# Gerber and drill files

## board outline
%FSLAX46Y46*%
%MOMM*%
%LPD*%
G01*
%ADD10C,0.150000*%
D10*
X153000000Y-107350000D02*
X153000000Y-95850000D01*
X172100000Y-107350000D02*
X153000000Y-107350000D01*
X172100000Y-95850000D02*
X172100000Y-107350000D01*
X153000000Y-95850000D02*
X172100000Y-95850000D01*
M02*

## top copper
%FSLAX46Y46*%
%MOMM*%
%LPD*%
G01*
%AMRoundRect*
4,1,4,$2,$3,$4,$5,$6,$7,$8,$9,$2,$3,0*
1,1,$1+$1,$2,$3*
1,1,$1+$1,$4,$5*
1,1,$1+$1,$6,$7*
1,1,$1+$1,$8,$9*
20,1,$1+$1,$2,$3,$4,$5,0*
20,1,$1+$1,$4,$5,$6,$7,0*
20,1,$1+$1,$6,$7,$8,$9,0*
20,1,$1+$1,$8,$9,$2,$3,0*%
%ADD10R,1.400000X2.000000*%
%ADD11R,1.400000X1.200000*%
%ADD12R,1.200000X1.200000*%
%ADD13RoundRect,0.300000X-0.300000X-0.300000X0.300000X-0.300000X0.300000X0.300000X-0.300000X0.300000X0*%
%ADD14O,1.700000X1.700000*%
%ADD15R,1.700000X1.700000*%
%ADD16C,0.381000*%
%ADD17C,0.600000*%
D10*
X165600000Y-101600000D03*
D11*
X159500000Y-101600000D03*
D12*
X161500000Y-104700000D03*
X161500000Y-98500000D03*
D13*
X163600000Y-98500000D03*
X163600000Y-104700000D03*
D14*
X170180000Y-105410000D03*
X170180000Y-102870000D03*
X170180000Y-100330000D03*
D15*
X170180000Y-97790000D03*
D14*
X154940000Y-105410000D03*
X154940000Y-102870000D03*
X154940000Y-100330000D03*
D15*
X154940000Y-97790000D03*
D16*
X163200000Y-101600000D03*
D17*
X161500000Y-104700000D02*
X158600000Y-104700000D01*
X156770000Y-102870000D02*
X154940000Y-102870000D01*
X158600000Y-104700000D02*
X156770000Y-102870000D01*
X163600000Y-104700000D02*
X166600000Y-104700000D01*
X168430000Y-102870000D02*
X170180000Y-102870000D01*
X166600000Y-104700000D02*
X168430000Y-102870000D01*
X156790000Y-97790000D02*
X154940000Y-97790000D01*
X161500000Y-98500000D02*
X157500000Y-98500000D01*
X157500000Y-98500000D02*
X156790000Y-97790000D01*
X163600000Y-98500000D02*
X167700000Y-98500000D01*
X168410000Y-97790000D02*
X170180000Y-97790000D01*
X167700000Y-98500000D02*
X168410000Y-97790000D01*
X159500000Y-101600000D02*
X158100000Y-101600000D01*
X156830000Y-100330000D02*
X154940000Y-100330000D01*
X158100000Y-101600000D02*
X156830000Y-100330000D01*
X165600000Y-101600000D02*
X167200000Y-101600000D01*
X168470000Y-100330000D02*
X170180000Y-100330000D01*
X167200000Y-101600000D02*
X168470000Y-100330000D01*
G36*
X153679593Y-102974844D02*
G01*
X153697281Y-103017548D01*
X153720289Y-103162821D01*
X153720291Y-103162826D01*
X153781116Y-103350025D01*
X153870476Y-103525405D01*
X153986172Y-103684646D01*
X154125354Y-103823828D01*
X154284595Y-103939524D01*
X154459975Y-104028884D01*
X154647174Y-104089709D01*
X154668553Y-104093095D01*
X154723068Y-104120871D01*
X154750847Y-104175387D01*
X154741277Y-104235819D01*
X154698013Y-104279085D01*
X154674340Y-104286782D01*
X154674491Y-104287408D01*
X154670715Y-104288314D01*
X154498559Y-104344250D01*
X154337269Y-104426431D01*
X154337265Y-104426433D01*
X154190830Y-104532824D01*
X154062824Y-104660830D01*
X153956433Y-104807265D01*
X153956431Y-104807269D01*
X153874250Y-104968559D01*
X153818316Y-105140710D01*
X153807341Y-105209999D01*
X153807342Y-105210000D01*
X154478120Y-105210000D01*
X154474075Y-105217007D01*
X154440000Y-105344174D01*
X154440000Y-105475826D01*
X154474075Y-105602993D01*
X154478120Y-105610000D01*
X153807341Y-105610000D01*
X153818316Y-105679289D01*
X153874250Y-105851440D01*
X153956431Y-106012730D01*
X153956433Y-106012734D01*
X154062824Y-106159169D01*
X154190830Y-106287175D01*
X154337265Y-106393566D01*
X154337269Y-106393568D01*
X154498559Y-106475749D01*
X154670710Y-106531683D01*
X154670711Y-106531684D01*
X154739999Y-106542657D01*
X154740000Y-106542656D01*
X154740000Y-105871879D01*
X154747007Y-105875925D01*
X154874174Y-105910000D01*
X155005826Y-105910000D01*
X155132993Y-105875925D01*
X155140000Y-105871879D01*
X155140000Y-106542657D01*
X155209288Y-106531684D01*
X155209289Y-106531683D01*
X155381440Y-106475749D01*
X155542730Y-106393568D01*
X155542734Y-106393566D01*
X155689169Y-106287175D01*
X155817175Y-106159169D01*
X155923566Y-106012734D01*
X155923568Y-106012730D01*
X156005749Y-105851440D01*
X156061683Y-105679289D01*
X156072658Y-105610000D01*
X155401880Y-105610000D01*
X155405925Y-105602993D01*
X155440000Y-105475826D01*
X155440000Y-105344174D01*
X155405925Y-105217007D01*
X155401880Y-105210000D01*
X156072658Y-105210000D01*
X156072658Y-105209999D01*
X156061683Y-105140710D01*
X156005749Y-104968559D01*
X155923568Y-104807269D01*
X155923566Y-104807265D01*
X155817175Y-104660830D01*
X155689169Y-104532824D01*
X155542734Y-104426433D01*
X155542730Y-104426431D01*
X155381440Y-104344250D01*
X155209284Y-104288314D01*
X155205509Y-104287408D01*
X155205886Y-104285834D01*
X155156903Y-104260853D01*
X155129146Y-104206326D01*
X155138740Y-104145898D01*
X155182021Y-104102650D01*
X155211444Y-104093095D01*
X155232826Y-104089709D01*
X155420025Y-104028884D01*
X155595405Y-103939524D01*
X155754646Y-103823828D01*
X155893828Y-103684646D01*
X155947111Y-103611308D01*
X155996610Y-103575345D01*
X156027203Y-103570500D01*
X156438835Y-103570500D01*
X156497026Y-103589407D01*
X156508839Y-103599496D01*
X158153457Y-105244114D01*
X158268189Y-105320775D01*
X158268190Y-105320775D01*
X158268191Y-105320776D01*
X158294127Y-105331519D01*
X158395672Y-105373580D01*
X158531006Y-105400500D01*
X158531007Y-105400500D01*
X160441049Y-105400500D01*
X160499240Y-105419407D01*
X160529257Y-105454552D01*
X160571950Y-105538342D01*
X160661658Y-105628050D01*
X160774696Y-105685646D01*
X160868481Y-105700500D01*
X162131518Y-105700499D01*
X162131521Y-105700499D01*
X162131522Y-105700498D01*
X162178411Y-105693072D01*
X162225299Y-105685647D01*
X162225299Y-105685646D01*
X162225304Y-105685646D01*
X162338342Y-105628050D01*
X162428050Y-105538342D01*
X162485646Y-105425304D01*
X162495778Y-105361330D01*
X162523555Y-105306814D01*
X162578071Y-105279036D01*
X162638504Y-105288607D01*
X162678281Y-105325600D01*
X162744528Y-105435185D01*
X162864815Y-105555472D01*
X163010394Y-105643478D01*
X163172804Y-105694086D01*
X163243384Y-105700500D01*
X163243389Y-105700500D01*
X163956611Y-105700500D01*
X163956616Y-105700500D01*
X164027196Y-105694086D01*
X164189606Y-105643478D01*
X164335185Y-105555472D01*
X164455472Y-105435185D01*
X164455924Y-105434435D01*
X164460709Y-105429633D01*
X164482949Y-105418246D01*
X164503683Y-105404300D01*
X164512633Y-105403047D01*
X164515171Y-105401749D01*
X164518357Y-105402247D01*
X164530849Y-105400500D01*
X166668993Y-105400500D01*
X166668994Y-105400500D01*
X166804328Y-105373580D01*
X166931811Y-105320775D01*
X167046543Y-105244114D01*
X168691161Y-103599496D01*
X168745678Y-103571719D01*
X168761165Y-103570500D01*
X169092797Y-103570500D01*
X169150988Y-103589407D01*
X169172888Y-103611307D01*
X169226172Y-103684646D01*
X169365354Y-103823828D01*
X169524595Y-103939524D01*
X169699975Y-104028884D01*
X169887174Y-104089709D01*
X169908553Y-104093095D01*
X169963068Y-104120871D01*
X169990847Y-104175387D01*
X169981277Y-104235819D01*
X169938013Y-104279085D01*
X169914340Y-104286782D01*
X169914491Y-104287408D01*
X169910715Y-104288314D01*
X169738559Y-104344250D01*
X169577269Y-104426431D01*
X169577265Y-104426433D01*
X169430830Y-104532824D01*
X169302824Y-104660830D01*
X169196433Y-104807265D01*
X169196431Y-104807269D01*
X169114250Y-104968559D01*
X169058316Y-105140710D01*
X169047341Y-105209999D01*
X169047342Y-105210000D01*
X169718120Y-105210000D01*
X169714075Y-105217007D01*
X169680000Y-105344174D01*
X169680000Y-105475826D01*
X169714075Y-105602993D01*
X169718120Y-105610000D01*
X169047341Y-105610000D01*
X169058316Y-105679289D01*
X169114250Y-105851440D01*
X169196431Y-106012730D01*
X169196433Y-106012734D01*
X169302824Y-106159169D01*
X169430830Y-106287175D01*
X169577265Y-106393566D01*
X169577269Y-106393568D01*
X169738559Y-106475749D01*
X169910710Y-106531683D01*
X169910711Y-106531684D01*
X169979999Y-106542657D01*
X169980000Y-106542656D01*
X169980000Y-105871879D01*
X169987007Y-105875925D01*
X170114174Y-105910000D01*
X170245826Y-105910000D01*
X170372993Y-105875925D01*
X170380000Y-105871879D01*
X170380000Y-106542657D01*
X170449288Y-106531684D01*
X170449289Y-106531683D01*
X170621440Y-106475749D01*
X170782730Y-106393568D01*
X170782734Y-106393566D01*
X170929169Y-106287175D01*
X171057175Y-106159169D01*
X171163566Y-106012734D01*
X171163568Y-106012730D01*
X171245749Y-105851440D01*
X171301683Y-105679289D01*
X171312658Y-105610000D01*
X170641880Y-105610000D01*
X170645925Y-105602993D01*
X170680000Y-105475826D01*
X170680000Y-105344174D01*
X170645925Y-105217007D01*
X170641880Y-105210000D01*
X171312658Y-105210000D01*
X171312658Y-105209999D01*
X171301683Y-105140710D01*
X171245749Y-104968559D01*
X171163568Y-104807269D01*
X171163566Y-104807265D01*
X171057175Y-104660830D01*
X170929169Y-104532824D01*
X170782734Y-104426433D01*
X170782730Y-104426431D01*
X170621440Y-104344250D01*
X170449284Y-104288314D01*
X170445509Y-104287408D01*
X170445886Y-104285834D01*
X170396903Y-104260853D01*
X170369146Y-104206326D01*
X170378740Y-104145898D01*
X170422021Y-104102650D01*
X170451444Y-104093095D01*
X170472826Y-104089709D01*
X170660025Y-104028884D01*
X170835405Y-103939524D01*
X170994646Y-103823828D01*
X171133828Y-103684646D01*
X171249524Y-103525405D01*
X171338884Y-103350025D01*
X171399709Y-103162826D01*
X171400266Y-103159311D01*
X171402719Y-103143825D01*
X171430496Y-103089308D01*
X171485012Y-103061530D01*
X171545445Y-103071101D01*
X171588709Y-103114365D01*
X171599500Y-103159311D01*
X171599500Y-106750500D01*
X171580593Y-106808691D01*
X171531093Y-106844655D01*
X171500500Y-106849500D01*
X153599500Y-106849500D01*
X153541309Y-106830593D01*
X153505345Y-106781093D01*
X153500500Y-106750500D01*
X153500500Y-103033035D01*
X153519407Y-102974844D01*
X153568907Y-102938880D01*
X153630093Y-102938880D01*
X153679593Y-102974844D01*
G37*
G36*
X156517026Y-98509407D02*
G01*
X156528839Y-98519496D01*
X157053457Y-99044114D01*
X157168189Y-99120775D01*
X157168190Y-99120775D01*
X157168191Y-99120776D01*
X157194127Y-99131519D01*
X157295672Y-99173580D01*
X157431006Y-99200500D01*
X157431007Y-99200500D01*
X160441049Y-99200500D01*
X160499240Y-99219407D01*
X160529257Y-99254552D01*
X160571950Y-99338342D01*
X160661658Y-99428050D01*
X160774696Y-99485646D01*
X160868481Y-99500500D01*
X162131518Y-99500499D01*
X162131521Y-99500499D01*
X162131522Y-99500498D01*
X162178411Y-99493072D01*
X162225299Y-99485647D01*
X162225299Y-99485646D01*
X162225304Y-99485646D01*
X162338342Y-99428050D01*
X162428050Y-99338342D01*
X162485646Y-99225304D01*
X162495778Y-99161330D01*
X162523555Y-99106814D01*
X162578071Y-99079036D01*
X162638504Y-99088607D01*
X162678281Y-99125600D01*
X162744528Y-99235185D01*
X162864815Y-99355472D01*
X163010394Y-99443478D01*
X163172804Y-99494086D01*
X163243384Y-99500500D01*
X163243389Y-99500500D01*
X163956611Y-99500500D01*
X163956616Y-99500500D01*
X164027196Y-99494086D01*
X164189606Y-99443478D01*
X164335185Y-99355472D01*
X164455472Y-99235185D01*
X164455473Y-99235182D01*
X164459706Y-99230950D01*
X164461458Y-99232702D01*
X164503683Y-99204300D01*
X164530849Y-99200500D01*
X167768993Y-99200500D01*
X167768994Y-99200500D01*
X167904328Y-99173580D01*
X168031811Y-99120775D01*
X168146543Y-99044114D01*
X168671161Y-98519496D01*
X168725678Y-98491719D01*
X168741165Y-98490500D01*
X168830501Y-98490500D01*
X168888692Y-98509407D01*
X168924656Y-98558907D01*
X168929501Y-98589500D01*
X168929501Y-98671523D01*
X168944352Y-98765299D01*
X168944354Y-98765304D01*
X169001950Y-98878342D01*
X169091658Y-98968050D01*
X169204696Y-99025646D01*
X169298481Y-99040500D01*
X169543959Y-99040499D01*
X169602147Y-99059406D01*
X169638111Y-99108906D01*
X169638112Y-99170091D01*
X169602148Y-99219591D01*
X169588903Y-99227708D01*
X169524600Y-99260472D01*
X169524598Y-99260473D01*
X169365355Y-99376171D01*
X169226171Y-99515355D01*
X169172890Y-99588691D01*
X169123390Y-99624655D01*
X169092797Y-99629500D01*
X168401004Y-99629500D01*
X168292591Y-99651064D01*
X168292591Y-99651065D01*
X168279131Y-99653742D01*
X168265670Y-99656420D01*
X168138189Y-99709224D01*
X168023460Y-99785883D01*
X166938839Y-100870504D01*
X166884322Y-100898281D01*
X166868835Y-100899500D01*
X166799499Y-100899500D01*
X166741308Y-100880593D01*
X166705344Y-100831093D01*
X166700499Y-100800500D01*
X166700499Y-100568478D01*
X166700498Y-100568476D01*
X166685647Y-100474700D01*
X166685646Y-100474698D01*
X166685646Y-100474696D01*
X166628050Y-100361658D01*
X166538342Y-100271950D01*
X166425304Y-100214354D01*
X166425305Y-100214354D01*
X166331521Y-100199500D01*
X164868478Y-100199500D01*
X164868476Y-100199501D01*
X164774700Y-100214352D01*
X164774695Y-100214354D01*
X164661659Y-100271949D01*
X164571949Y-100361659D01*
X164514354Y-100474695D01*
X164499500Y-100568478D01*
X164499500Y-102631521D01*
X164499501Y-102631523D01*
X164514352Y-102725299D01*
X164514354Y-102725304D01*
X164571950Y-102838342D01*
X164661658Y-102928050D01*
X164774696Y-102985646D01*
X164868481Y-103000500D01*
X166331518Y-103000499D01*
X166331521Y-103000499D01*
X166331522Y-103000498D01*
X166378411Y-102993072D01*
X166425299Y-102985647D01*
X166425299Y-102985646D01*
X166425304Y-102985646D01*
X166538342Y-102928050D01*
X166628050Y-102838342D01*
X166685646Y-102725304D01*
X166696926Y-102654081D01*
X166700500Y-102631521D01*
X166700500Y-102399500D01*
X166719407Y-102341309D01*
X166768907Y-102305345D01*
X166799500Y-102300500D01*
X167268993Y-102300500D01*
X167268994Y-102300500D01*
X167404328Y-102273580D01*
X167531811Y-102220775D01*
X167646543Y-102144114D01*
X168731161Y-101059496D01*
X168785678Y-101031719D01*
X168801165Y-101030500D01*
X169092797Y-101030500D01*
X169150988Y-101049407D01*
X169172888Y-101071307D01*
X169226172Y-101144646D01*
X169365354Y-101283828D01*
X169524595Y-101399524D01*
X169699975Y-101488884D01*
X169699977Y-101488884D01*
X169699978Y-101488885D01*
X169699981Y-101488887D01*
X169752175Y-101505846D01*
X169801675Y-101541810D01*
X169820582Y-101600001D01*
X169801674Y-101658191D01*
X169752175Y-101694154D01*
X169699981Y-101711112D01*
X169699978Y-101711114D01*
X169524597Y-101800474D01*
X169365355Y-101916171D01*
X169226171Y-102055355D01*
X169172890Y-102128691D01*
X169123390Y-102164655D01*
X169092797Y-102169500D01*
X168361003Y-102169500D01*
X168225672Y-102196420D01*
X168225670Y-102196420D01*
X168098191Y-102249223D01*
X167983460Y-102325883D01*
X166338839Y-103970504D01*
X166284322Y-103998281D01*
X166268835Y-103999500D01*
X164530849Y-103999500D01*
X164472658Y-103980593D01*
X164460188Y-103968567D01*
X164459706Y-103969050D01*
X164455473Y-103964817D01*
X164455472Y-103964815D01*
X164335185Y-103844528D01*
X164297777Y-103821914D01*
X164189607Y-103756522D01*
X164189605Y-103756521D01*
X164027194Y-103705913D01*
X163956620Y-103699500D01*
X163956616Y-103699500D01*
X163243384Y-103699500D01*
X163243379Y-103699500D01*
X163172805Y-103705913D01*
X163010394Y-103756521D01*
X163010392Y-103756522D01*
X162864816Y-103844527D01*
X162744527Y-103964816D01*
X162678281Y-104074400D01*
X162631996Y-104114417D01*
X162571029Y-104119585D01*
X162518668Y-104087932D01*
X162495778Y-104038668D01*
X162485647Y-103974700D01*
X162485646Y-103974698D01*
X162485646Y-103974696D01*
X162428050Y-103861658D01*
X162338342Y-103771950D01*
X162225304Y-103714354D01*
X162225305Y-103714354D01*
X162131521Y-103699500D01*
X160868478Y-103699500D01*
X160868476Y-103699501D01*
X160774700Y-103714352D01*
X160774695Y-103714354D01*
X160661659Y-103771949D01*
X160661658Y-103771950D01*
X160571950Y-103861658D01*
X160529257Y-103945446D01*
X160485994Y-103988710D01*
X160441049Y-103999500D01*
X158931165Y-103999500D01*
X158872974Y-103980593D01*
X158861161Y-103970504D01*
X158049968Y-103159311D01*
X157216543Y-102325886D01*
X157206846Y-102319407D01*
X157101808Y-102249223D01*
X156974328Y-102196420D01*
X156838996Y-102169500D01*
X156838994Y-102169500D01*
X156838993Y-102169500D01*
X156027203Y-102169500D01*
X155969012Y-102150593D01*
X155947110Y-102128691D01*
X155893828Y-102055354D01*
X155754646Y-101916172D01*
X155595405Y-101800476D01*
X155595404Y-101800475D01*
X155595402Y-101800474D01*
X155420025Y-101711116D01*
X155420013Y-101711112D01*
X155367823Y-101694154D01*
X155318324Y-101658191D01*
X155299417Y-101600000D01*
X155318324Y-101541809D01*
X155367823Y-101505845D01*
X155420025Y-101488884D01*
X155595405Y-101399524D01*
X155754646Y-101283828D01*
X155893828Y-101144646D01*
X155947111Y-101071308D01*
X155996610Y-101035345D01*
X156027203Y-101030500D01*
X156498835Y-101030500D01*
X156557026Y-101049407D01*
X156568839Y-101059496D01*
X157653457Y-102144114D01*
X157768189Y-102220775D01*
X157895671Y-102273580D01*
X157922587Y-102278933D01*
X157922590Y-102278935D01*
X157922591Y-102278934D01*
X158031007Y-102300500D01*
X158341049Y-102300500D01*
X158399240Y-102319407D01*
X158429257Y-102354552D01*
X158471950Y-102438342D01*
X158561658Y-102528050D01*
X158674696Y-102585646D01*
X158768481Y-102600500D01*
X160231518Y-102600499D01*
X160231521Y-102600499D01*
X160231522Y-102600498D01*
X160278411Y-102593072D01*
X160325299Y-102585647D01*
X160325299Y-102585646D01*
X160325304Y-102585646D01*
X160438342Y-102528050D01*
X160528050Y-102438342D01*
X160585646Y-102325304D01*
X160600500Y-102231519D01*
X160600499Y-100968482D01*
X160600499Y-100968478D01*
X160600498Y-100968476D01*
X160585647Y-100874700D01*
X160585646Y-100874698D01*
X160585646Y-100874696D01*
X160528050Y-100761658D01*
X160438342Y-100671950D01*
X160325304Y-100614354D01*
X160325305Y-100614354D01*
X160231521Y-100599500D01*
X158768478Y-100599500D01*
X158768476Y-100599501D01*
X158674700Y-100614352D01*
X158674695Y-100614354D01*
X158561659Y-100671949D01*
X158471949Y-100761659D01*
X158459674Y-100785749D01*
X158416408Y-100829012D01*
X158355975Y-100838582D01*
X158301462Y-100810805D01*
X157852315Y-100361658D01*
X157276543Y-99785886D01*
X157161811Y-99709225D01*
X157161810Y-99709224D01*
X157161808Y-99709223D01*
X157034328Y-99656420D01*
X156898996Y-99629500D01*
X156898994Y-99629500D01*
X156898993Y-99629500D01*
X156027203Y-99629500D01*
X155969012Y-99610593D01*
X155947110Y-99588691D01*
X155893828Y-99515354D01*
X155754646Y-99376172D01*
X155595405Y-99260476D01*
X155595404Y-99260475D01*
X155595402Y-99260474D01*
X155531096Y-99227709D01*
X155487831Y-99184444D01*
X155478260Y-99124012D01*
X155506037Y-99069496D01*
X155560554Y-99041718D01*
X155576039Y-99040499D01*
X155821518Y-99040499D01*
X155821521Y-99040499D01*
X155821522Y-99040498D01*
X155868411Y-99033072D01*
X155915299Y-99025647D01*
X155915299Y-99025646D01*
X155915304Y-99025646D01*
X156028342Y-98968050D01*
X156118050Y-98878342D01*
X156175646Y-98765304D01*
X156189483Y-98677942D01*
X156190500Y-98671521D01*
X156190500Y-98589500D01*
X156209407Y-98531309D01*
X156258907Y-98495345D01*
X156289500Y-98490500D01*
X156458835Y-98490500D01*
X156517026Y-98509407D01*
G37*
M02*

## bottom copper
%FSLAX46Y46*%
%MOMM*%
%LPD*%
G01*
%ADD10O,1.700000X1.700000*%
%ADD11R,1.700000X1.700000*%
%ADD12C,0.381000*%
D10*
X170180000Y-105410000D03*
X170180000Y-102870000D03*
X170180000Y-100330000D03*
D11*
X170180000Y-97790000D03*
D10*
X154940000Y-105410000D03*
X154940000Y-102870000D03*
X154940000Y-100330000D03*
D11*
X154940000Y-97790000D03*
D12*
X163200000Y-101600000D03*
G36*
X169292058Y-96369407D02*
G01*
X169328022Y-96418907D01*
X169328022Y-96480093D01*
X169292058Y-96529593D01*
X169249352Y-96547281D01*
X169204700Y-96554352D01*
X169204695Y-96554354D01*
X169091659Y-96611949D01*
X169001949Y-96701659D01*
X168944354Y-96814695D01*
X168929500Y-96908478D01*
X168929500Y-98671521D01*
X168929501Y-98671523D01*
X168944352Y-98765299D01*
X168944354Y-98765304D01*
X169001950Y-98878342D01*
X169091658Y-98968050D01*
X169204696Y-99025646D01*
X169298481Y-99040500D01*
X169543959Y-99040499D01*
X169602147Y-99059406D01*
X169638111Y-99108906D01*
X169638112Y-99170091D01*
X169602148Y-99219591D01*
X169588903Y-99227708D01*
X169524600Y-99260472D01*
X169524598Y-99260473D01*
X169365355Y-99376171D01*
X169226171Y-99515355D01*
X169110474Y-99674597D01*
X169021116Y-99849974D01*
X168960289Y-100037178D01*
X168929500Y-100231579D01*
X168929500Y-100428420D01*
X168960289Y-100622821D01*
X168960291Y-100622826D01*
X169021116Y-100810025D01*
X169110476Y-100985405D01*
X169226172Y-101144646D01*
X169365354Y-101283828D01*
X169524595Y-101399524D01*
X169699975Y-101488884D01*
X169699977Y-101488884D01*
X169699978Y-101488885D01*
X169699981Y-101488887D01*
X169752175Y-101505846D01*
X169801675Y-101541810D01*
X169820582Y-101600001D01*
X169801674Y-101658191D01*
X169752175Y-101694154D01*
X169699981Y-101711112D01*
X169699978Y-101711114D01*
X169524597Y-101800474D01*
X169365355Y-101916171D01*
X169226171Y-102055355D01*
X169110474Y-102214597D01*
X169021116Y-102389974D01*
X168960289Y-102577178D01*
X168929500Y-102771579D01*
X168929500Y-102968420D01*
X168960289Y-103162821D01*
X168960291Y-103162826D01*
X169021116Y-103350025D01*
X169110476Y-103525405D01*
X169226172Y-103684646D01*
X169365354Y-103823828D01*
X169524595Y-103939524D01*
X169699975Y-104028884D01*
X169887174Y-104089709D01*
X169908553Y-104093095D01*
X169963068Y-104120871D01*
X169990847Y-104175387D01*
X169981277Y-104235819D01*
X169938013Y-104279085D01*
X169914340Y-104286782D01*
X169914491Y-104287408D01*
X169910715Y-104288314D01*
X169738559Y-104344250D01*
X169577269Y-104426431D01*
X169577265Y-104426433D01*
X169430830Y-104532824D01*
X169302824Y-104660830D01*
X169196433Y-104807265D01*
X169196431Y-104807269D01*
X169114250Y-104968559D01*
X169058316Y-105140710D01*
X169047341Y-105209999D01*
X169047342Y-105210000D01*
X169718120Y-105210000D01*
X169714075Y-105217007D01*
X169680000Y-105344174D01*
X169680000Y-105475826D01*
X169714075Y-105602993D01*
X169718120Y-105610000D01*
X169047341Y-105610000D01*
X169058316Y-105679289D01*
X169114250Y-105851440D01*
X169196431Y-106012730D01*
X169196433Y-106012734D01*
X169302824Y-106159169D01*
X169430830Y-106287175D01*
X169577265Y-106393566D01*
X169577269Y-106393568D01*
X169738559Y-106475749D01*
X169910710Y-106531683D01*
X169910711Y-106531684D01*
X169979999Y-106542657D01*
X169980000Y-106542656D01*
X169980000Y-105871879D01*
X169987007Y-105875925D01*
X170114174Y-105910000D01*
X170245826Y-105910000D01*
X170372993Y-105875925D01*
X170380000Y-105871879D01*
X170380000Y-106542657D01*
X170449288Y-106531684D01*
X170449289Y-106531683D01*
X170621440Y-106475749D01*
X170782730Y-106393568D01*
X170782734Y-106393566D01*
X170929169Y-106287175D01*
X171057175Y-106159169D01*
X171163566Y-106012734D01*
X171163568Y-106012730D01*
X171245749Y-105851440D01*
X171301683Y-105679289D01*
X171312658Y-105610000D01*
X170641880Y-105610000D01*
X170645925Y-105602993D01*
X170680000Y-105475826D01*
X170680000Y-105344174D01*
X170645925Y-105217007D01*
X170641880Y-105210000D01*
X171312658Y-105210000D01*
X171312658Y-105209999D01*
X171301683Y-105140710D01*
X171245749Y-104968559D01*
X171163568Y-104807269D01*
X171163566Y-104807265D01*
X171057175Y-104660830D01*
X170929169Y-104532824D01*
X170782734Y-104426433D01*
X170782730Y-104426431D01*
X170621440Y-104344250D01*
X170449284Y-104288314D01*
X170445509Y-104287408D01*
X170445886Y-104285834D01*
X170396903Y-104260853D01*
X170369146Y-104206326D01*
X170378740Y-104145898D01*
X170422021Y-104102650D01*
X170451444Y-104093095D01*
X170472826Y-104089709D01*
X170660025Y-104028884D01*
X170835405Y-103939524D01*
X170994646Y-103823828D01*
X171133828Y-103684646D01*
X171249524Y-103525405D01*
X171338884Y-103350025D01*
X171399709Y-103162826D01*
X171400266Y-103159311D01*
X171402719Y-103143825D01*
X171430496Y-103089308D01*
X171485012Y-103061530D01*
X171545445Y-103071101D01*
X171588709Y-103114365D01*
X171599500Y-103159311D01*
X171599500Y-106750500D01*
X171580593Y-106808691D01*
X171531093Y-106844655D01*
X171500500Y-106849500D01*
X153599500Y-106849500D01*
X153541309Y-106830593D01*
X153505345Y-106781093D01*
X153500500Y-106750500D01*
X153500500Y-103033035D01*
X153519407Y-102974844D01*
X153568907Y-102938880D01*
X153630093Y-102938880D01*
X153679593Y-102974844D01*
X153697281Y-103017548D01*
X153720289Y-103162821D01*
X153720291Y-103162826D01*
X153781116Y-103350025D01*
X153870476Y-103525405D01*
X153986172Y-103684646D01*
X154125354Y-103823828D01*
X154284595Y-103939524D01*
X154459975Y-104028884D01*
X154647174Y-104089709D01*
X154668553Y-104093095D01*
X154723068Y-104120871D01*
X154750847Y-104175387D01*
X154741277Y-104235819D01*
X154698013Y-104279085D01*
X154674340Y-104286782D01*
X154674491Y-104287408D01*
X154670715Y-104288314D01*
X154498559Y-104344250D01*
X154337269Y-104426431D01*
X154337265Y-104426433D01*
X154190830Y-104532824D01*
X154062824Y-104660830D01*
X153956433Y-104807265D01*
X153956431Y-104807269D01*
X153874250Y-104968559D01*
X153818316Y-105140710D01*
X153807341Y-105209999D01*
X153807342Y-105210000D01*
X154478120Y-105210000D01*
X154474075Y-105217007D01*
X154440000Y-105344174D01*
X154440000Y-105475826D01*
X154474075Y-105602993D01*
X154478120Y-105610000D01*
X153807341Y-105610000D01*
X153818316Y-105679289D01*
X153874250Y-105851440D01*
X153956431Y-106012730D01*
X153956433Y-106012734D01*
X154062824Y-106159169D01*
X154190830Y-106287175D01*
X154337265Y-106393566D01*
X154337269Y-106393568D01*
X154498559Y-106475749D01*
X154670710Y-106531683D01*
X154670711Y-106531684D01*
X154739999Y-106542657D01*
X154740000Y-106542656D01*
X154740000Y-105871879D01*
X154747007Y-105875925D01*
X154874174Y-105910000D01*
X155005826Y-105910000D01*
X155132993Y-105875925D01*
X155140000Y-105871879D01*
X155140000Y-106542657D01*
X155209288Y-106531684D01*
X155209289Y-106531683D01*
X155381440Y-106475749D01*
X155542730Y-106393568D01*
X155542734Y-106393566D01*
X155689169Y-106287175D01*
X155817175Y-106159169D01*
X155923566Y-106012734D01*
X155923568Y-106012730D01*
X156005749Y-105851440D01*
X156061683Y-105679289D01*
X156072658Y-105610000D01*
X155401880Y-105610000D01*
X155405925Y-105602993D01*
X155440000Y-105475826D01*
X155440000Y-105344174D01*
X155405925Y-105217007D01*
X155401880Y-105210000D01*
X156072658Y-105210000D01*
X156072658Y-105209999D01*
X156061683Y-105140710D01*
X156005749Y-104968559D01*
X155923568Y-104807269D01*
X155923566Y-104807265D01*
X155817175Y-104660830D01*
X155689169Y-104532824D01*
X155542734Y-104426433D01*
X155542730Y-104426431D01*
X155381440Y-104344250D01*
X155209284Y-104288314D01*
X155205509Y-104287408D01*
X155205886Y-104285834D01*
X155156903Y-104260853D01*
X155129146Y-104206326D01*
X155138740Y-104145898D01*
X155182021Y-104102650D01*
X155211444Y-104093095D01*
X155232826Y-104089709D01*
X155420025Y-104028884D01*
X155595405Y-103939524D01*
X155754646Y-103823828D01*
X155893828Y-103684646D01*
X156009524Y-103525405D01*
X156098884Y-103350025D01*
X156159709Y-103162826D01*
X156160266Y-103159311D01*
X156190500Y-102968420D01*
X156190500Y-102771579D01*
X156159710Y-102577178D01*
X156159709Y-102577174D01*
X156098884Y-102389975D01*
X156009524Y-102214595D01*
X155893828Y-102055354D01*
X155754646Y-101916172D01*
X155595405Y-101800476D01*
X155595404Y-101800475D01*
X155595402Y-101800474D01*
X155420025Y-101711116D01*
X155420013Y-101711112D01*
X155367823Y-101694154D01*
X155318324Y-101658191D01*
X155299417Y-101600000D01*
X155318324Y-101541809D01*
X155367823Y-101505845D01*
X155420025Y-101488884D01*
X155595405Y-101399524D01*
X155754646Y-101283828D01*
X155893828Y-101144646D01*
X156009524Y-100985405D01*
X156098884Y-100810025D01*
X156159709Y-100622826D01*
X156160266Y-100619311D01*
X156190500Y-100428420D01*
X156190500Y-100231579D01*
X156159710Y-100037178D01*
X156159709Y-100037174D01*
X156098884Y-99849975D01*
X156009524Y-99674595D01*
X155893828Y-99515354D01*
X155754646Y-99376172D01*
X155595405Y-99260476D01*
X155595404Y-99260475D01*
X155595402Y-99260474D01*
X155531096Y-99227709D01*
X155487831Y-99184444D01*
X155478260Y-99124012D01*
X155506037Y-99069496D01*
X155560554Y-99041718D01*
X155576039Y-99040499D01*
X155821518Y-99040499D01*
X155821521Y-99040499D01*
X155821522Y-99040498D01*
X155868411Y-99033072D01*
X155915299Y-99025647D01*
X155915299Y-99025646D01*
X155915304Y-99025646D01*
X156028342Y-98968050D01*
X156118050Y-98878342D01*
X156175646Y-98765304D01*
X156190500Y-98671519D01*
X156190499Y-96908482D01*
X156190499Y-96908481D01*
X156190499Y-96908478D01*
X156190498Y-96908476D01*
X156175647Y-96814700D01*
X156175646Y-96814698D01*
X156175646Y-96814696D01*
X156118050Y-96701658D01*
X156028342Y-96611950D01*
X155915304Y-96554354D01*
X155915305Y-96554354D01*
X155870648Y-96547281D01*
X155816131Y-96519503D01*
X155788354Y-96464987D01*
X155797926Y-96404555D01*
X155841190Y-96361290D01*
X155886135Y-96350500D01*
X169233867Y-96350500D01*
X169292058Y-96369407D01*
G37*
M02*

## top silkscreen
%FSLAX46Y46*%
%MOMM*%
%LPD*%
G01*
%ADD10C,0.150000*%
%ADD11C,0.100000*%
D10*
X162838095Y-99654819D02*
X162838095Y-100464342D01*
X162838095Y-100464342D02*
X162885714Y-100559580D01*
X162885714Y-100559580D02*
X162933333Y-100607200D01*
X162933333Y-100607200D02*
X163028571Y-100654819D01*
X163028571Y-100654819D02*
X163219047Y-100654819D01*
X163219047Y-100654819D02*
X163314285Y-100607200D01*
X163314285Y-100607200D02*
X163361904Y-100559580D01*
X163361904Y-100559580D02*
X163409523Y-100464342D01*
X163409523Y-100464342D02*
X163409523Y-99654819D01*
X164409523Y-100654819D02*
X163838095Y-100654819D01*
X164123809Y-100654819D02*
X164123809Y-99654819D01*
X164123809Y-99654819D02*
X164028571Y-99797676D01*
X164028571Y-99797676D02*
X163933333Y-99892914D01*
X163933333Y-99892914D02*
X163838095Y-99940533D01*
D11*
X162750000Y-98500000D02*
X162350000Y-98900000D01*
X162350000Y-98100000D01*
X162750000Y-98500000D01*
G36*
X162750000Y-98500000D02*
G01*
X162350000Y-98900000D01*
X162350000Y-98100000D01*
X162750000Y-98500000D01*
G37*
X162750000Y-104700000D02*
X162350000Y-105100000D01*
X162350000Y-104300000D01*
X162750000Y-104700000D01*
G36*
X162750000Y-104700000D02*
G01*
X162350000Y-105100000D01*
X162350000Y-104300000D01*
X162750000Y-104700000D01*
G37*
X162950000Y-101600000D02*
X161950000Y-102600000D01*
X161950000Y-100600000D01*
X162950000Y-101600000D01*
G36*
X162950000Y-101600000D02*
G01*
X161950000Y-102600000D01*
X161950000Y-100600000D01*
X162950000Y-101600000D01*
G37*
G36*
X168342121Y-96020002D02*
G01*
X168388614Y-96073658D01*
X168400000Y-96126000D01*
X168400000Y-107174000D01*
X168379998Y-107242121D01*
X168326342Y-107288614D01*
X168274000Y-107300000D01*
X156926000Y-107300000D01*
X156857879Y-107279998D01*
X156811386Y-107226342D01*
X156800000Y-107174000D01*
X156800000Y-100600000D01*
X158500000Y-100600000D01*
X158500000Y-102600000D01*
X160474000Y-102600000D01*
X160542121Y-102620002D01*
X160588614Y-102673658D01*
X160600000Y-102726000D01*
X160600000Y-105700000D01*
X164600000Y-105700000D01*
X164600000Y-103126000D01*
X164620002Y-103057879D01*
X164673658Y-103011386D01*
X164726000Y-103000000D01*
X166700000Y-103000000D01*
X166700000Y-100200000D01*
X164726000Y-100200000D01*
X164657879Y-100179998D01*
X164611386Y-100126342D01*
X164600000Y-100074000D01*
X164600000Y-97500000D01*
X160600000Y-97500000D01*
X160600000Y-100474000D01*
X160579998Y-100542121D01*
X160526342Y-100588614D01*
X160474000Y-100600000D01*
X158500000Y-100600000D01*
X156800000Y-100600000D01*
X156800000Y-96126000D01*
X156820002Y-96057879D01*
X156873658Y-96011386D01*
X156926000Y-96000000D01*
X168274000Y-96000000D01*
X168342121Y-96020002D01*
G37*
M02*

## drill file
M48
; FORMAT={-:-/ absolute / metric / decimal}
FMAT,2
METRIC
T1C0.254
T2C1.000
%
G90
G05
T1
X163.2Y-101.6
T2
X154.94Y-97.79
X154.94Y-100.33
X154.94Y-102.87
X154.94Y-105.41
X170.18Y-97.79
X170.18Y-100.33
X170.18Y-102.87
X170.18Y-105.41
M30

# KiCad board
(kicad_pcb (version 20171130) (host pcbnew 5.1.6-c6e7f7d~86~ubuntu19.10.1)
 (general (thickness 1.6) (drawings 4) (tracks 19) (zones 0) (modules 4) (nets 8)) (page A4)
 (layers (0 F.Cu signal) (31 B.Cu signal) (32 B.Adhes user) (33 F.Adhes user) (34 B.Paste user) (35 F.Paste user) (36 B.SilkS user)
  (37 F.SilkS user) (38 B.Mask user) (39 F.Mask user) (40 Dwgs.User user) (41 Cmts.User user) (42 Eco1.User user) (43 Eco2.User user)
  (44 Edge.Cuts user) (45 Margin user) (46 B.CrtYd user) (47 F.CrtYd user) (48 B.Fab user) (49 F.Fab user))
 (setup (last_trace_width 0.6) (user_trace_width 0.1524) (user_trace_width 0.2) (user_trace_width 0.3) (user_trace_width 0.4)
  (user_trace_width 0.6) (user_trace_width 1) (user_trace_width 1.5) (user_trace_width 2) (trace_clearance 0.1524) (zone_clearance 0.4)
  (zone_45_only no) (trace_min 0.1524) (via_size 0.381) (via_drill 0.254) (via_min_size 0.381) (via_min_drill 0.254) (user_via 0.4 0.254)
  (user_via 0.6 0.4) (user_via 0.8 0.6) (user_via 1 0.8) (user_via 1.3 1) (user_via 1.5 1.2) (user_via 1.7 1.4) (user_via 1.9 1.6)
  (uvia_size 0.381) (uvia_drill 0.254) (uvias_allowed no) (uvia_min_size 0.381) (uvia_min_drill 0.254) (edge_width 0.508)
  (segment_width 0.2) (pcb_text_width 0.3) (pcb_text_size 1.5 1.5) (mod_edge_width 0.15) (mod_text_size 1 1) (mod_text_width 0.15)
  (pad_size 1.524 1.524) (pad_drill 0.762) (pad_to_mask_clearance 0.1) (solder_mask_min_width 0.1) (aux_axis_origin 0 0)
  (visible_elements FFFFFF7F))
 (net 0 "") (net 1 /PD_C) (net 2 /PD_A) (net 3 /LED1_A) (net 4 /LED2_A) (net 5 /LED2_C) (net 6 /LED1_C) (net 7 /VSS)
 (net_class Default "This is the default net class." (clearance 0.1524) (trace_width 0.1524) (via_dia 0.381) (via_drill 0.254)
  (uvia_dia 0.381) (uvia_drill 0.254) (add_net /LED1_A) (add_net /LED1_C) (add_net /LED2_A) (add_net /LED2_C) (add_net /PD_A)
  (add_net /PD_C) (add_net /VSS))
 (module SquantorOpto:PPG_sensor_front (layer F.Cu) (at 162.55 101.6)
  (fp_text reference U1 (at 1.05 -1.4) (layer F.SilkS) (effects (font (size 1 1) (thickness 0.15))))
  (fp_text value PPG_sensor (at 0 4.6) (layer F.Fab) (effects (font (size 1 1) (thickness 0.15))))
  (fp_poly (pts (xy 0.2 -3.1) (xy -0.2 -2.7) (xy -0.2 -3.5)) (layer F.SilkS) (width 0.1))
  (fp_poly (pts (xy 0.2 3.1) (xy -0.2 3.5) (xy -0.2 2.7)) (layer F.SilkS) (width 0.1))
  (fp_poly (pts (xy 0.4 0) (xy -0.6 1) (xy -0.6 -1)) (layer F.SilkS) (width 0.1))
  (pad 5 smd rect (at 3.05 0) (size 1.4 2) (layers F.Cu F.Paste F.Mask) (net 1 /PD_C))
  (pad 2 smd rect (at -3.05 0) (size 1.4 1.2) (layers F.Cu F.Paste F.Mask) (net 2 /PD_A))
  (pad 1 smd rect (at -1.05 3.1) (size 1.2 1.2) (layers F.Cu F.Paste F.Mask) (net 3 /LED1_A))
  (pad 3 smd rect (at -1.05 -3.1) (size 1.2 1.2) (layers F.Cu F.Paste F.Mask) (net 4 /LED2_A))
  (pad 4 smd roundrect (at 1.05 -3.1) (size 1.2 1.2) (layers F.Cu F.Paste F.Mask) (roundrect_rratio 0.25) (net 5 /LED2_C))
  (pad 6 smd roundrect (at 1.05 3.1) (size 1.2 1.2) (layers F.Cu F.Paste F.Mask) (roundrect_rratio 0.25) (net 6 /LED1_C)))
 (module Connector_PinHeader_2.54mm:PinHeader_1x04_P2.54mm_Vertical (layer B.Cu) (at 170.18 97.79 180)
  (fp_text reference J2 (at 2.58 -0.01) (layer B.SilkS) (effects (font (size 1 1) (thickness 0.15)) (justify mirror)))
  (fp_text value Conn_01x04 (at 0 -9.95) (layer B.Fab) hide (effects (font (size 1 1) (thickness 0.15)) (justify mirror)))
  (pad 4 thru_hole oval (at 0 -7.62 180) (size 1.7 1.7) (drill 1) (layers *.Cu *.Mask) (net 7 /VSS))
  (pad 3 thru_hole oval (at 0 -5.08 180) (size 1.7 1.7) (drill 1) (layers *.Cu *.Mask) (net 6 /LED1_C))
  (pad 2 thru_hole oval (at 0 -2.54 180) (size 1.7 1.7) (drill 1) (layers *.Cu *.Mask) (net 1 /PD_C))
  (pad 1 thru_hole rect (at 0 0 180) (size 1.7 1.7) (drill 1) (layers *.Cu *.Mask) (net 5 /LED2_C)))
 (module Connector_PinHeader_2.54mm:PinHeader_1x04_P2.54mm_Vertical (layer B.Cu) (at 154.94 97.79 180)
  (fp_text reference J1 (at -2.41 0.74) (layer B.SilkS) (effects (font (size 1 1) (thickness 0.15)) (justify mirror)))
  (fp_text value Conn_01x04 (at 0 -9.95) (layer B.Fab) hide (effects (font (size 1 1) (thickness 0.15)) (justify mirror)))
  (pad 4 thru_hole oval (at 0 -7.62 180) (size 1.7 1.7) (drill 1) (layers *.Cu *.Mask) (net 7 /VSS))
  (pad 3 thru_hole oval (at 0 -5.08 180) (size 1.7 1.7) (drill 1) (layers *.Cu *.Mask) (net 3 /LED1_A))
  (pad 2 thru_hole oval (at 0 -2.54 180) (size 1.7 1.7) (drill 1) (layers *.Cu *.Mask) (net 2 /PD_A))
  (pad 1 thru_hole rect (at 0 0 180) (size 1.7 1.7) (drill 1) (layers *.Cu *.Mask) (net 4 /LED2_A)))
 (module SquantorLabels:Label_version (layer B.Cu) (at 157.25 102.6 90)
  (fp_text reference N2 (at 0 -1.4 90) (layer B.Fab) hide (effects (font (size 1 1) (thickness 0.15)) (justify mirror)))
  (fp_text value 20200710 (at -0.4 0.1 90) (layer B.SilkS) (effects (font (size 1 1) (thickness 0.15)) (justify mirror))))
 (gr_line (start 153 107.35) (end 153 95.85) (layer Edge.Cuts) (width 0.15))
 (gr_line (start 172.1 107.35) (end 153 107.35) (layer Edge.Cuts) (width 0.15))
 (gr_line (start 172.1 95.85) (end 172.1 107.35) (layer Edge.Cuts) (width 0.15))
 (gr_line (start 153 95.85) (end 172.1 95.85) (layer Edge.Cuts) (width 0.15))
 (segment (start 161.5 104.7) (end 158.6 104.7) (width 0.6) (layer F.Cu) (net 3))
 (segment (start 156.77 102.87) (end 154.94 102.87) (width 0.6) (layer F.Cu) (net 3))
 (segment (start 158.6 104.7) (end 156.77 102.87) (width 0.6) (layer F.Cu) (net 3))
 (segment (start 163.6 104.7) (end 166.6 104.7) (width 0.6) (layer F.Cu) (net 6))
 (segment (start 168.43 102.87) (end 170.18 102.87) (width 0.6) (layer F.Cu) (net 6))
 (segment (start 166.6 104.7) (end 168.43 102.87) (width 0.6) (layer F.Cu) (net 6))
 (segment (start 156.79 97.79) (end 154.94 97.79) (width 0.6) (layer F.Cu) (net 4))
 (segment (start 161.5 98.5) (end 157.5 98.5) (width 0.6) (layer F.Cu) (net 4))
 (segment (start 157.5 98.5) (end 156.79 97.79) (width 0.6) (layer F.Cu) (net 4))
 (segment (start 163.6 98.5) (end 167.7 98.5) (width 0.6) (layer F.Cu) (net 5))
 (segment (start 168.41 97.79) (end 170.18 97.79) (width 0.6) (layer F.Cu) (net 5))
 (segment (start 167.7 98.5) (end 168.41 97.79) (width 0.6) (layer F.Cu) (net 5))
 (segment (start 159.5 101.6) (end 158.1 101.6) (width 0.6) (layer F.Cu) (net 2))
 (segment (start 156.83 100.33) (end 154.94 100.33) (width 0.6) (layer F.Cu) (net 2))
 (segment (start 158.1 101.6) (end 156.83 100.33) (width 0.6) (layer F.Cu) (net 2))
 (segment (start 165.6 101.6) (end 167.2 101.6) (width 0.6) (layer F.Cu) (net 1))
 (segment (start 168.47 100.33) (end 170.18 100.33) (width 0.6) (layer F.Cu) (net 1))
 (segment (start 167.2 101.6) (end 168.47 100.33) (width 0.6) (layer F.Cu) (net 1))
 (via (at 163.2 101.6) (size 0.381) (drill 0.254) (layers F.Cu B.Cu) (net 7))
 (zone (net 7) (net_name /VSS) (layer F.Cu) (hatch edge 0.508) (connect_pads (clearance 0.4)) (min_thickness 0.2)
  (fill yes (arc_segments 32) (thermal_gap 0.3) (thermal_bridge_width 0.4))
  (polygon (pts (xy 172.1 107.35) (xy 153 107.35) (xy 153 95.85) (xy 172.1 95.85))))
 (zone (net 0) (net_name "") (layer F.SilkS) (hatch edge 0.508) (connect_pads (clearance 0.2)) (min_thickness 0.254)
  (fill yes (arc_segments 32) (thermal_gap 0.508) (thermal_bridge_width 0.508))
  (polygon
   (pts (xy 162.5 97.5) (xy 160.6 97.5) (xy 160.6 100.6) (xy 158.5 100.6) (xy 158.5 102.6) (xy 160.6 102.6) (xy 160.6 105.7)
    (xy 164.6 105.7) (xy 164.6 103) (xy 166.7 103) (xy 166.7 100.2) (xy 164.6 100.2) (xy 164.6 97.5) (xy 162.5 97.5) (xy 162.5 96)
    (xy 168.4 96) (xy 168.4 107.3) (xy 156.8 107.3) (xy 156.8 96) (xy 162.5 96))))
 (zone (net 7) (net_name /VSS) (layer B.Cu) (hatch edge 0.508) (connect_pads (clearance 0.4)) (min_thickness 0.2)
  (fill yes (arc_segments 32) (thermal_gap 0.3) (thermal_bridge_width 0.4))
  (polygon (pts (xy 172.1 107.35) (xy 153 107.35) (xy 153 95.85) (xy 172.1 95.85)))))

